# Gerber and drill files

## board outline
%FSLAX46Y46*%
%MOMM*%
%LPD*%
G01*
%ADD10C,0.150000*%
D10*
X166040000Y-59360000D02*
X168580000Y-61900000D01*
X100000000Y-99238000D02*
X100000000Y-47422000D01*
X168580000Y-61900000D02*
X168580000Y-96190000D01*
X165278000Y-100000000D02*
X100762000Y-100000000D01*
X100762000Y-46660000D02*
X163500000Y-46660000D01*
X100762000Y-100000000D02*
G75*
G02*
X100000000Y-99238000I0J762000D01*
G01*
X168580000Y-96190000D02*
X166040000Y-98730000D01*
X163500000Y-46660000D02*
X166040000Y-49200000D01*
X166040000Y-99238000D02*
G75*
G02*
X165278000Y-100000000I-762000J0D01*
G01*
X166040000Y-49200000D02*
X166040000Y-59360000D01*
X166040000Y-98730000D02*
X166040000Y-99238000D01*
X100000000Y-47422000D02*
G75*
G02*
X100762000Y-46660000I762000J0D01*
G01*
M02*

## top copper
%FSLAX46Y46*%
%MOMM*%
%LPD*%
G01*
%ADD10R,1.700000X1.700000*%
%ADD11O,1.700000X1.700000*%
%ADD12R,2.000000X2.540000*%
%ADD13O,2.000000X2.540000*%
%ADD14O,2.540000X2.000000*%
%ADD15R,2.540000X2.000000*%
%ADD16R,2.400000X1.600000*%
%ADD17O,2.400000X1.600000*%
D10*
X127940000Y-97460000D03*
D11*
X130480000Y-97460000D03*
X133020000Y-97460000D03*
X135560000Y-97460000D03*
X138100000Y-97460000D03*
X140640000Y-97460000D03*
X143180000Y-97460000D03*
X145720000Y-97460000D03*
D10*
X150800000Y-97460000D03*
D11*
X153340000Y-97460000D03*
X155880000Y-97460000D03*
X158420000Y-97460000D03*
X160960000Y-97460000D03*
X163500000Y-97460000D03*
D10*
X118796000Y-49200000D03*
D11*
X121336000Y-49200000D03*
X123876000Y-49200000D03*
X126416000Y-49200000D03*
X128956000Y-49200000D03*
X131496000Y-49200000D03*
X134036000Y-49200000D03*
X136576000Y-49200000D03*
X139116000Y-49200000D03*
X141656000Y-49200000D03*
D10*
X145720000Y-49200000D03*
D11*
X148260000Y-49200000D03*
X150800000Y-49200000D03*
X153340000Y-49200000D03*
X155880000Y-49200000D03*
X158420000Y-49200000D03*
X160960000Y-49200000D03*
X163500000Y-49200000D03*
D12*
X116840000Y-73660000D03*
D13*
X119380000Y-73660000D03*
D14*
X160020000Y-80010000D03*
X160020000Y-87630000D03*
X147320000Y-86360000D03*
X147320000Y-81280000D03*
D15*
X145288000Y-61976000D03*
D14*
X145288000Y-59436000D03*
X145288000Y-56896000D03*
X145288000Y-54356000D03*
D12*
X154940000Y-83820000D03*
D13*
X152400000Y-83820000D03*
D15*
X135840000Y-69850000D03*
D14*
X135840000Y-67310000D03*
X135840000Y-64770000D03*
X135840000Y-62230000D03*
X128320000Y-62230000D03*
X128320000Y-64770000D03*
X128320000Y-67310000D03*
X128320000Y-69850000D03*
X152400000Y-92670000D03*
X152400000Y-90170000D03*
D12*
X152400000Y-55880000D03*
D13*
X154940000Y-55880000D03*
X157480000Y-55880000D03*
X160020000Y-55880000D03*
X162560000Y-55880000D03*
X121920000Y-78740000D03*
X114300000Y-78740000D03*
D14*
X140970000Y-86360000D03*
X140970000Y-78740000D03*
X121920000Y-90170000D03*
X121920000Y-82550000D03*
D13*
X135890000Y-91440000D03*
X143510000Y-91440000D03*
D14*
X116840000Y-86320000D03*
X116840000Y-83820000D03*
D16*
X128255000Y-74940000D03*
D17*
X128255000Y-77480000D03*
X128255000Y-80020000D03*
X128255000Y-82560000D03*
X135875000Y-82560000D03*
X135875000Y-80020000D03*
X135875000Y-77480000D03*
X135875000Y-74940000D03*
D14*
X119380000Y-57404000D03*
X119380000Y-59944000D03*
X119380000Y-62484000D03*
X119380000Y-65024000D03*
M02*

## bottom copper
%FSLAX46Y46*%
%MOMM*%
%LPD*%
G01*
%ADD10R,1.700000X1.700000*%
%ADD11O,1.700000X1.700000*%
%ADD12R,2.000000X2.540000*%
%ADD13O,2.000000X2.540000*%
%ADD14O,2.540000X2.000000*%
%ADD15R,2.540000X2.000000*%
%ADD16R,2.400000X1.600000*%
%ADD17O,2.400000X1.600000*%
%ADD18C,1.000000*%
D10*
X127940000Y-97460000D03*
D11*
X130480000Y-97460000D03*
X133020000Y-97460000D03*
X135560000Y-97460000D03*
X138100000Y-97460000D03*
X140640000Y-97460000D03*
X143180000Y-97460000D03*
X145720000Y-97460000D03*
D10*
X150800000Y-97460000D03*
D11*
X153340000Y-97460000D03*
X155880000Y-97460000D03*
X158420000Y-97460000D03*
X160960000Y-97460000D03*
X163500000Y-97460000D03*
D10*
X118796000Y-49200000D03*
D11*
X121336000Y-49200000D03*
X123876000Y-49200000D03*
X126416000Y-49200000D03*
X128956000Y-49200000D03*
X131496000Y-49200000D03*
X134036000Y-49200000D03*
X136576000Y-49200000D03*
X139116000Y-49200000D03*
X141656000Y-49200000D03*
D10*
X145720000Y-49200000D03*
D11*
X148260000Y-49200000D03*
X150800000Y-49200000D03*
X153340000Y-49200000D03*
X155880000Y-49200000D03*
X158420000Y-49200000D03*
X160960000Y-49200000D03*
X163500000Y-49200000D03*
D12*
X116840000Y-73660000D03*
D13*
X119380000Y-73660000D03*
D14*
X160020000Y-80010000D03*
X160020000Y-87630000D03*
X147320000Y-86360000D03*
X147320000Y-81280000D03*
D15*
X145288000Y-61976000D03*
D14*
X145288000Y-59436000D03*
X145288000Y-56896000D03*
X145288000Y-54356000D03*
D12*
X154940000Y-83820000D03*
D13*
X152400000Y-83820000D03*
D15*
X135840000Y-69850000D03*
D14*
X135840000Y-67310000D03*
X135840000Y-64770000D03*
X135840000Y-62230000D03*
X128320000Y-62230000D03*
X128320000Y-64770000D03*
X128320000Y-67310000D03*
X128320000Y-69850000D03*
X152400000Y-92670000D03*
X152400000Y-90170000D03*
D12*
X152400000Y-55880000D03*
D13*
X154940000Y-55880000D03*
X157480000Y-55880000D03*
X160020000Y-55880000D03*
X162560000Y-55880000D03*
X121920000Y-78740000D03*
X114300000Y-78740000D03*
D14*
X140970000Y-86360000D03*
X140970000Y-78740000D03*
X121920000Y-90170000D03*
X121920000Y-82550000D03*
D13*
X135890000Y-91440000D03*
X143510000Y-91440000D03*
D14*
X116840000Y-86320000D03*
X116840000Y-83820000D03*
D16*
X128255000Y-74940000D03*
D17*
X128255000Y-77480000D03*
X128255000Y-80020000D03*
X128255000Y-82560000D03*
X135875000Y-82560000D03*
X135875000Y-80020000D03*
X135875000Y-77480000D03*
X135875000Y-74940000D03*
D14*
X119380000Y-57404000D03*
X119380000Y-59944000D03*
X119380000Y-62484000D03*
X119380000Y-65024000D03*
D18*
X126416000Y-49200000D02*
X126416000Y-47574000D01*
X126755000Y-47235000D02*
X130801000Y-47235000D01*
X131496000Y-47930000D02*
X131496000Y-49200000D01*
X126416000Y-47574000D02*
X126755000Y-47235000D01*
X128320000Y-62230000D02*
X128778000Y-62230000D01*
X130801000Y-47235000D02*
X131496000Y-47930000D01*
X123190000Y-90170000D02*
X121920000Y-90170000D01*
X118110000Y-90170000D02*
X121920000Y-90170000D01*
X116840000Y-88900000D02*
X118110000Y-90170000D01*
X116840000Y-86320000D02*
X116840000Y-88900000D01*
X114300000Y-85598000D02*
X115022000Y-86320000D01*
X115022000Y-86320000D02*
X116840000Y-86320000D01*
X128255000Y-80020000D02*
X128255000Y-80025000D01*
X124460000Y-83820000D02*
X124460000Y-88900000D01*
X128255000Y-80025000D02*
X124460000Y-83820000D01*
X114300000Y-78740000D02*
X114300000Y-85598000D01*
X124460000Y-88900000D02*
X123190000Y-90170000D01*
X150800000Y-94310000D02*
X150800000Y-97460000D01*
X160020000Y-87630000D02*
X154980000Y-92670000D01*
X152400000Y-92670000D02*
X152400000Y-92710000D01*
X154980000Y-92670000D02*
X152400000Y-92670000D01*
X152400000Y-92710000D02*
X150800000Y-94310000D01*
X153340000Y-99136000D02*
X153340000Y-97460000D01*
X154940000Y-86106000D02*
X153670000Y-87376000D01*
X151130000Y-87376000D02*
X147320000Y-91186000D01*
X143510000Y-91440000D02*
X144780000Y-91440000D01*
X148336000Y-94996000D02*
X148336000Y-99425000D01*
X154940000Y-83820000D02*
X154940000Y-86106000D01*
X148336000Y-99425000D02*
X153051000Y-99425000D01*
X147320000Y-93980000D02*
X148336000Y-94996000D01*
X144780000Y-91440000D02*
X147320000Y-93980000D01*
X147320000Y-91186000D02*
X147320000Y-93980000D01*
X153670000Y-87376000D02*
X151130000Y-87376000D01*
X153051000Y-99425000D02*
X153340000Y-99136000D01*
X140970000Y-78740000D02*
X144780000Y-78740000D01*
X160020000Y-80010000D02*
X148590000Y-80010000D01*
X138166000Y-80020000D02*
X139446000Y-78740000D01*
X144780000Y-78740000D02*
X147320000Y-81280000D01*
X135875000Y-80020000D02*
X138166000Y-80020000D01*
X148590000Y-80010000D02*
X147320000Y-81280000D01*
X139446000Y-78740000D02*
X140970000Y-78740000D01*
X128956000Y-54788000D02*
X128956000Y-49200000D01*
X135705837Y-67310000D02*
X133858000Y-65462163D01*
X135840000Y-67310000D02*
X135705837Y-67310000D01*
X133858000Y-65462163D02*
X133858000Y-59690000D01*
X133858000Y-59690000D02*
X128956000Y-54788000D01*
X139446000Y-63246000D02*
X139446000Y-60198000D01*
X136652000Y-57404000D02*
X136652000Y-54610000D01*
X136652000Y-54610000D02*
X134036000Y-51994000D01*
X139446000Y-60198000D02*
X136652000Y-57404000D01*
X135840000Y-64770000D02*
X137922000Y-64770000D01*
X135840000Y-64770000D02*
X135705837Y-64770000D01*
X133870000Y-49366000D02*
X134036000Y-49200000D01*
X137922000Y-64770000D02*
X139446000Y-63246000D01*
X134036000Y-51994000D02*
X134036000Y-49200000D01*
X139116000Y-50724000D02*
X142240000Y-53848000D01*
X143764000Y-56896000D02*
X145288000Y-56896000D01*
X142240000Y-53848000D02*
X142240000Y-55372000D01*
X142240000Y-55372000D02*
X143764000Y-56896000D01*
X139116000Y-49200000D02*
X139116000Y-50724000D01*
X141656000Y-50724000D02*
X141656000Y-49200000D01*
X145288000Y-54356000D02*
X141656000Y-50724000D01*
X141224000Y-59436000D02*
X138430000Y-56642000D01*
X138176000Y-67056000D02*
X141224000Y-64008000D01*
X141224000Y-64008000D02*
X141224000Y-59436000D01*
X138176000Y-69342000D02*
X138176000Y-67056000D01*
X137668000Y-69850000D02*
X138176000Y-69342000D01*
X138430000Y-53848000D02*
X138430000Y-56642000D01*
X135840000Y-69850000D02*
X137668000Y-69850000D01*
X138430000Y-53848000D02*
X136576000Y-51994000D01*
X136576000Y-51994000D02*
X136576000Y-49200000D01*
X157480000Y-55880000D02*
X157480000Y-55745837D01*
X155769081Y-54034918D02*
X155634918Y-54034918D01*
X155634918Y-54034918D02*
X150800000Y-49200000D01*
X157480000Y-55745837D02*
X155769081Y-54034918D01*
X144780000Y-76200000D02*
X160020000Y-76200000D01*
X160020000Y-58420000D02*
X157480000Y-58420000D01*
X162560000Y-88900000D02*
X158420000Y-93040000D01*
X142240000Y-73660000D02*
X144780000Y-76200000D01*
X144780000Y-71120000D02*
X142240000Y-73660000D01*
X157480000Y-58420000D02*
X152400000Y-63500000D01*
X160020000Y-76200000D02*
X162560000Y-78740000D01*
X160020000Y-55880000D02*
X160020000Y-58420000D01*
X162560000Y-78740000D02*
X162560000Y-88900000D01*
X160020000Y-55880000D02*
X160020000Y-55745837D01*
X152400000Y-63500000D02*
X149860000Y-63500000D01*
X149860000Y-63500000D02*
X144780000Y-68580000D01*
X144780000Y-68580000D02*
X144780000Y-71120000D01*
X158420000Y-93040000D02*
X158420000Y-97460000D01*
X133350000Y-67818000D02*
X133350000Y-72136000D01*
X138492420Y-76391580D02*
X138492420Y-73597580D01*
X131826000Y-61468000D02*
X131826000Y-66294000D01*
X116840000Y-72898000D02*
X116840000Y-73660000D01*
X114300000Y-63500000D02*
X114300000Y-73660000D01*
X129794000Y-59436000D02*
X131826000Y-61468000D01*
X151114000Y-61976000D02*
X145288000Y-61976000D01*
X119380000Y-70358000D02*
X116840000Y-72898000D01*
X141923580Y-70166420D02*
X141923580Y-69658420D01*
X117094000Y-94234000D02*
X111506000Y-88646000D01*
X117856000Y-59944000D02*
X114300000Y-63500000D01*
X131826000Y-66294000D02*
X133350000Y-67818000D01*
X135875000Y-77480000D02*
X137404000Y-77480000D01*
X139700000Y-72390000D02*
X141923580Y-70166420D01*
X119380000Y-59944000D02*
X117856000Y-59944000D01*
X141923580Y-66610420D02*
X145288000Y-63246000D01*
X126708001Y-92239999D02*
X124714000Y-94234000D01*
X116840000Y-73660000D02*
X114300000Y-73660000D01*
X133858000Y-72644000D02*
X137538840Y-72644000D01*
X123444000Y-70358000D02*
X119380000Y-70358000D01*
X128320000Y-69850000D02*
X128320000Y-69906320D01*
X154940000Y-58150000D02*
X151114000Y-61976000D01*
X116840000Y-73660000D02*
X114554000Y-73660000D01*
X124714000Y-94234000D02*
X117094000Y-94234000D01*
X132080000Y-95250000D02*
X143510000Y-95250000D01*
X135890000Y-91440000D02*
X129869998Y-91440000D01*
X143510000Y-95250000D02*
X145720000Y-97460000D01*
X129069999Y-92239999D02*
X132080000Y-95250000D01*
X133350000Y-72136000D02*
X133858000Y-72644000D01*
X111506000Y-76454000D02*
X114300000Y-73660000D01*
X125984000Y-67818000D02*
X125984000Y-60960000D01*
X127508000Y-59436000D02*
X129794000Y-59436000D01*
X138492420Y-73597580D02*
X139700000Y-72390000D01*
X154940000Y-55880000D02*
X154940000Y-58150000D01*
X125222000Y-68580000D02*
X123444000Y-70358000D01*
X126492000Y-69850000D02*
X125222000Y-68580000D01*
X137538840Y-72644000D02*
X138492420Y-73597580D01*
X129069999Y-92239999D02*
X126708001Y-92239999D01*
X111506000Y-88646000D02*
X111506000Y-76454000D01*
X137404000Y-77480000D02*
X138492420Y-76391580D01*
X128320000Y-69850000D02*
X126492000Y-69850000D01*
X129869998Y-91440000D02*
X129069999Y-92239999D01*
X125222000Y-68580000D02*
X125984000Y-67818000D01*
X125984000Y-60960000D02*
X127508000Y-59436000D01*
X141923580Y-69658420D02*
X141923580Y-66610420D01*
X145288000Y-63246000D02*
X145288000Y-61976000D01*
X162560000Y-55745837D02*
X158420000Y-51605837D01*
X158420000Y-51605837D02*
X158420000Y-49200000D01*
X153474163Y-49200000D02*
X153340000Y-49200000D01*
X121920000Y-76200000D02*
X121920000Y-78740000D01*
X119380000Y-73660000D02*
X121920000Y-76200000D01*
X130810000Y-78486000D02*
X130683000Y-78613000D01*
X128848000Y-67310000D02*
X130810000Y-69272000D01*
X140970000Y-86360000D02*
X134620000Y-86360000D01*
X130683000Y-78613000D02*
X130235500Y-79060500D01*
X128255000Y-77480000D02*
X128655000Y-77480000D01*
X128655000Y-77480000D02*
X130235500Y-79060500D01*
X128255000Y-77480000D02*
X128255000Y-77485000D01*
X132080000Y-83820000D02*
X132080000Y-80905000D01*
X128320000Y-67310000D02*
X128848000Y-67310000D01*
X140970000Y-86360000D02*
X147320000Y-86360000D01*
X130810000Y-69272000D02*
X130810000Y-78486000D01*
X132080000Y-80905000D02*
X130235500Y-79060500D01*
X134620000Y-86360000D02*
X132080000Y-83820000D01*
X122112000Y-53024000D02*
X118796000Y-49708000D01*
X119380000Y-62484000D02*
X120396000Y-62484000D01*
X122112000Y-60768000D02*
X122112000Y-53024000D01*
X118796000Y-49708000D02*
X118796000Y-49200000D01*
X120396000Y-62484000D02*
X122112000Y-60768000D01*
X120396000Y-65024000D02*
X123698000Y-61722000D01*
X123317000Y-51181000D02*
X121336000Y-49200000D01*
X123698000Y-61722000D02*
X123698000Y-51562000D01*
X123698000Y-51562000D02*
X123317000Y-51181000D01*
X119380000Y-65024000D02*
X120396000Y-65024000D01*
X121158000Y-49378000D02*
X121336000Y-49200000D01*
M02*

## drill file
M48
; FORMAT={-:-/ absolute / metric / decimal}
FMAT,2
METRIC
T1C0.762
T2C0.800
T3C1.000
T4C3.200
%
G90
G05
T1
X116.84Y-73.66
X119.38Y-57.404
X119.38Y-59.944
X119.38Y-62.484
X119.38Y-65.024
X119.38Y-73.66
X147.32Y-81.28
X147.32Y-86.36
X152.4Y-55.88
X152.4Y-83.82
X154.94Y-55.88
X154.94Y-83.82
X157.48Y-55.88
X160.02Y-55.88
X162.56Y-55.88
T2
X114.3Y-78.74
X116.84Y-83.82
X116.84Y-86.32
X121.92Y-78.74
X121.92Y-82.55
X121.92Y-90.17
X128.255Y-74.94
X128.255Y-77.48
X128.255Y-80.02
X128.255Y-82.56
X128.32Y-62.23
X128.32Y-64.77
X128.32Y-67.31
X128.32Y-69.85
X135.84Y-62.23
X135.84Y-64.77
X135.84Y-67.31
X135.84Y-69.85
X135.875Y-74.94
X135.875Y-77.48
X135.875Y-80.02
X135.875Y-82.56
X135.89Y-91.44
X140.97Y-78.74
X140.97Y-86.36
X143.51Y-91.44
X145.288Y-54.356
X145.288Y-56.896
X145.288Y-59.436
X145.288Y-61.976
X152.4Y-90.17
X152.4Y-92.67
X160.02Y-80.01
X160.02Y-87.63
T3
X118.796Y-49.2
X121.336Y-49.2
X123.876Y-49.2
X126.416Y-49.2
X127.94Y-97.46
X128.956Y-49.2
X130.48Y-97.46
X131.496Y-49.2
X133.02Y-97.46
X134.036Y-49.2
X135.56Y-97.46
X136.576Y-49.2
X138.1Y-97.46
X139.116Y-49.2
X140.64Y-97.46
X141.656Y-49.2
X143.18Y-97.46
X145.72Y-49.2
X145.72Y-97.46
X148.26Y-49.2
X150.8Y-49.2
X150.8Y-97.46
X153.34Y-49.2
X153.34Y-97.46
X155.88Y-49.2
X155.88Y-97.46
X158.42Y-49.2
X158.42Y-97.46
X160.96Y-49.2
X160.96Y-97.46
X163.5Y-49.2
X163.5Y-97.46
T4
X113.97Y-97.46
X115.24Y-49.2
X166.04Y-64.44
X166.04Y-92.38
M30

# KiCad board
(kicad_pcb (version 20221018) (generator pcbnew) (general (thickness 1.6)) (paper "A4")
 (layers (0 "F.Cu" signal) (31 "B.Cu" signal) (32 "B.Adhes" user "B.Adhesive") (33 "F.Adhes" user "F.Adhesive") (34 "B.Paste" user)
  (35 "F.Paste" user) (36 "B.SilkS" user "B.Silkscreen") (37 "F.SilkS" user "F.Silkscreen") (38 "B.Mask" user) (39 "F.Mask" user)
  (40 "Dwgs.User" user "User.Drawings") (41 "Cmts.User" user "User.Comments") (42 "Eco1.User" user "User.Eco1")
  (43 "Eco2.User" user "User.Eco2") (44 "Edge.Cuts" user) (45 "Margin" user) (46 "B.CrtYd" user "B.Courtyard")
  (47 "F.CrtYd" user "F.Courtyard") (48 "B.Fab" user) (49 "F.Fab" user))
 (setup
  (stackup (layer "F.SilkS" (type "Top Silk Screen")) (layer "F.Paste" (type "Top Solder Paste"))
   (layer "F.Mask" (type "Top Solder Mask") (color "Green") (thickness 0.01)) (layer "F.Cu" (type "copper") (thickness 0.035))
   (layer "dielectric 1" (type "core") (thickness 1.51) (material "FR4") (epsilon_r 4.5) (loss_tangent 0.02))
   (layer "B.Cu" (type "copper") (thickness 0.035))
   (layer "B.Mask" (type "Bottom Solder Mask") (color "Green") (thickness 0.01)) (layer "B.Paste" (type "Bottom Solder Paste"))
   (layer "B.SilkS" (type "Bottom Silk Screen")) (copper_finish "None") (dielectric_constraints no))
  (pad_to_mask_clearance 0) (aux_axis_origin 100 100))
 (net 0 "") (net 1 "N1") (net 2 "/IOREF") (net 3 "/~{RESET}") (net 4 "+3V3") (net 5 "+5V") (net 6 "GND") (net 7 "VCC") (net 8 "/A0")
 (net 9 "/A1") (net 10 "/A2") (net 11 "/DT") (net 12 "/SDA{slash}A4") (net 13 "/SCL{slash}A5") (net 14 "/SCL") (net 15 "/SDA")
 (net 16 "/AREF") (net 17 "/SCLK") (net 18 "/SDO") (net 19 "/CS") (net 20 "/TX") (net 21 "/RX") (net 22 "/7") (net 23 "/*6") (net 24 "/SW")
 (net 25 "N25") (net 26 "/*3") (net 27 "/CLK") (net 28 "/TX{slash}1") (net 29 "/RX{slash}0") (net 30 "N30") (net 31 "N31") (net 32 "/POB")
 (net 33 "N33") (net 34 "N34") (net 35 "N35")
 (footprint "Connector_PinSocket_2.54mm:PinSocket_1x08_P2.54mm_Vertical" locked (layer "F.Cu") (at 127.94 97.46 90)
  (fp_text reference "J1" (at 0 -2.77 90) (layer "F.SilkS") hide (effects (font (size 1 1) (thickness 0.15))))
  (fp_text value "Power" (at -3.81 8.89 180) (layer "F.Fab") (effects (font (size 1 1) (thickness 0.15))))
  (pad "1" thru_hole rect locked (at 0 0 90) (size 1.7 1.7) (drill 1) (layers "*.Cu" "*.Mask") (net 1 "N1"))
  (pad "2" thru_hole oval locked (at 0 2.54 90) (size 1.7 1.7) (drill 1) (layers "*.Cu" "*.Mask") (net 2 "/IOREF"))
  (pad "3" thru_hole oval locked (at 0 5.08 90) (size 1.7 1.7) (drill 1) (layers "*.Cu" "*.Mask") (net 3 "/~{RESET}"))
  (pad "4" thru_hole oval locked (at 0 7.62 90) (size 1.7 1.7) (drill 1) (layers "*.Cu" "*.Mask") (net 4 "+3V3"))
  (pad "5" thru_hole oval locked (at 0 10.16 90) (size 1.7 1.7) (drill 1) (layers "*.Cu" "*.Mask") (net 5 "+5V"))
  (pad "6" thru_hole oval locked (at 0 12.7 90) (size 1.7 1.7) (drill 1) (layers "*.Cu" "*.Mask") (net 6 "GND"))
  (pad "7" thru_hole oval locked (at 0 15.24 90) (size 1.7 1.7) (drill 1) (layers "*.Cu" "*.Mask") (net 6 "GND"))
  (pad "8" thru_hole oval locked (at 0 17.78 90) (size 1.7 1.7) (drill 1) (layers "*.Cu" "*.Mask") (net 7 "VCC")))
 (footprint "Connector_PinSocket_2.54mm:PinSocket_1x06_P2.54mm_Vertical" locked (layer "F.Cu") (at 150.8 97.46 90)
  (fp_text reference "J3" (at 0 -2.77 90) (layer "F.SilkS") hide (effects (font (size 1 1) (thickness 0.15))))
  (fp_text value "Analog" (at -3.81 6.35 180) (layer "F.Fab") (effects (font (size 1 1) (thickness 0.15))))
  (pad "1" thru_hole rect locked (at 0 0 90) (size 1.7 1.7) (drill 1) (layers "*.Cu" "*.Mask") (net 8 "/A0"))
  (pad "2" thru_hole oval locked (at 0 2.54 90) (size 1.7 1.7) (drill 1) (layers "*.Cu" "*.Mask") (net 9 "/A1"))
  (pad "3" thru_hole oval locked (at 0 5.08 90) (size 1.7 1.7) (drill 1) (layers "*.Cu" "*.Mask") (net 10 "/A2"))
  (pad "4" thru_hole oval locked (at 0 7.62 90) (size 1.7 1.7) (drill 1) (layers "*.Cu" "*.Mask") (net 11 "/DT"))
  (pad "5" thru_hole oval locked (at 0 10.16 90) (size 1.7 1.7) (drill 1) (layers "*.Cu" "*.Mask") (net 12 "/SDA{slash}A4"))
  (pad "6" thru_hole oval locked (at 0 12.7 90) (size 1.7 1.7) (drill 1) (layers "*.Cu" "*.Mask") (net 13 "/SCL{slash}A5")))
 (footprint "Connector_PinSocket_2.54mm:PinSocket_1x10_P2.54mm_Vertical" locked (layer "F.Cu") (at 118.796 49.2 90)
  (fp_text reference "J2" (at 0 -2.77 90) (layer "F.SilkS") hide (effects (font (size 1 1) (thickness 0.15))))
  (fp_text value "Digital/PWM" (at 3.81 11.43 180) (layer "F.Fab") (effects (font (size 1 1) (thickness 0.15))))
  (pad "1" thru_hole rect locked (at 0 0 90) (size 1.7 1.7) (drill 1) (layers "*.Cu" "*.Mask") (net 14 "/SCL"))
  (pad "2" thru_hole oval locked (at 0 2.54 90) (size 1.7 1.7) (drill 1) (layers "*.Cu" "*.Mask") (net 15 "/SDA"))
  (pad "3" thru_hole oval locked (at 0 5.08 90) (size 1.7 1.7) (drill 1) (layers "*.Cu" "*.Mask") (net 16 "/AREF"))
  (pad "4" thru_hole oval locked (at 0 7.62 90) (size 1.7 1.7) (drill 1) (layers "*.Cu" "*.Mask") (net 6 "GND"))
  (pad "5" thru_hole oval locked (at 0 10.16 90) (size 1.7 1.7) (drill 1) (layers "*.Cu" "*.Mask") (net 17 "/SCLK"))
  (pad "6" thru_hole oval locked (at 0 12.7 90) (size 1.7 1.7) (drill 1) (layers "*.Cu" "*.Mask") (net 6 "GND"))
  (pad "7" thru_hole oval locked (at 0 15.24 90) (size 1.7 1.7) (drill 1) (layers "*.Cu" "*.Mask") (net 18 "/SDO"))
  (pad "8" thru_hole oval locked (at 0 17.78 90) (size 1.7 1.7) (drill 1) (layers "*.Cu" "*.Mask") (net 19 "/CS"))
  (pad "9" thru_hole oval locked (at 0 20.32 90) (size 1.7 1.7) (drill 1) (layers "*.Cu" "*.Mask") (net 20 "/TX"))
  (pad "10" thru_hole oval locked (at 0 22.86 90) (size 1.7 1.7) (drill 1) (layers "*.Cu" "*.Mask") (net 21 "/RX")))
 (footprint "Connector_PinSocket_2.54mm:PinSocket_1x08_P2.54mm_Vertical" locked (layer "F.Cu") (at 145.72 49.2 90)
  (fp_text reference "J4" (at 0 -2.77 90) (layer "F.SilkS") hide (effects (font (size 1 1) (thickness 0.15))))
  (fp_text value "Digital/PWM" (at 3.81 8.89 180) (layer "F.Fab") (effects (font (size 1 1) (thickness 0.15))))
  (pad "1" thru_hole rect locked (at 0 0 90) (size 1.7 1.7) (drill 1) (layers "*.Cu" "*.Mask") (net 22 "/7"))
  (pad "2" thru_hole oval locked (at 0 2.54 90) (size 1.7 1.7) (drill 1) (layers "*.Cu" "*.Mask") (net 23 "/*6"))
  (pad "3" thru_hole oval locked (at 0 5.08 90) (size 1.7 1.7) (drill 1) (layers "*.Cu" "*.Mask") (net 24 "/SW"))
  (pad "4" thru_hole oval locked (at 0 7.62 90) (size 1.7 1.7) (drill 1) (layers "*.Cu" "*.Mask") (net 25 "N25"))
  (pad "5" thru_hole oval locked (at 0 10.16 90) (size 1.7 1.7) (drill 1) (layers "*.Cu" "*.Mask") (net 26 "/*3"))
  (pad "6" thru_hole oval locked (at 0 12.7 90) (size 1.7 1.7) (drill 1) (layers "*.Cu" "*.Mask") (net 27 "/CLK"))
  (pad "7" thru_hole oval locked (at 0 15.24 90) (size 1.7 1.7) (drill 1) (layers "*.Cu" "*.Mask") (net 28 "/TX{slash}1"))
  (pad "8" thru_hole oval locked (at 0 17.78 90) (size 1.7 1.7) (drill 1) (layers "*.Cu" "*.Mask") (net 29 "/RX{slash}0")))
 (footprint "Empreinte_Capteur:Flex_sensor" (layer "F.Cu") (at 119.38 71.12)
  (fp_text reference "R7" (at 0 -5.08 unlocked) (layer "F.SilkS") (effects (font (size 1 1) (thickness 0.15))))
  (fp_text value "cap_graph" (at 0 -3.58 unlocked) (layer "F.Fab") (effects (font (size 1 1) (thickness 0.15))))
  (pad "1" thru_hole rect (at -2.54 2.54) (size 2 2.54) (drill 0.762) (layers "*.Cu" "*.Mask") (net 7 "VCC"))
  (pad "2" thru_hole oval (at 0 2.54) (size 2 2.54) (drill 0.762) (layers "*.Cu" "*.Mask") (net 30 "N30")))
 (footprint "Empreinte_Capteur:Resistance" (layer "F.Cu") (at 160.02 80.01 -90)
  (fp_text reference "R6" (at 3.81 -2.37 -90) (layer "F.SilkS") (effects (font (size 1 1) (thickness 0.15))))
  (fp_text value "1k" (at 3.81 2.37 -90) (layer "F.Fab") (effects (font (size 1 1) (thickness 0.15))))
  (pad "1" thru_hole oval (at 0 0 270) (size 2 2.54) (drill 0.8) (layers "*.Cu" "*.Mask") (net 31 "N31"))
  (pad "2" thru_hole oval (at 7.62 0 270) (size 2 2.54) (drill 0.8) (layers "*.Cu" "*.Mask") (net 8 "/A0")))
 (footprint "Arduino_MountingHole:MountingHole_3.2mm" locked (layer "F.Cu") (at 115.24 49.2)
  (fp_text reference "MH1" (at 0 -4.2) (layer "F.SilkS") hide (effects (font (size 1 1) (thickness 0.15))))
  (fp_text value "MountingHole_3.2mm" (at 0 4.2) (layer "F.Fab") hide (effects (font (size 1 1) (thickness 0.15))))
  (pad "" np_thru_hole circle locked (at 0 0) (size 3.2 3.2) (drill 3.2) (layers "*.Cu" "*.Mask")))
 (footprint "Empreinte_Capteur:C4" (layer "F.Cu") (at 144.78 83.82 90)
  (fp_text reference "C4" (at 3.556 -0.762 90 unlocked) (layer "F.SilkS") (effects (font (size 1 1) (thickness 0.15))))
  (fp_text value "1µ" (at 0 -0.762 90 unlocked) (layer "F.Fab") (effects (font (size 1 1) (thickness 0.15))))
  (pad "1" thru_hole oval (at -2.54 2.54 90) (size 2 2.54) (drill 0.762) (layers "*.Cu" "*.Mask") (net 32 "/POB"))
  (pad "2" thru_hole oval (at 2.54 2.54 90) (size 2 2.54) (drill 0.762) (layers "*.Cu" "*.Mask") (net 31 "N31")))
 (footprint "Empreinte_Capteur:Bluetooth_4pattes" (layer "F.Cu") (at 145.288 58.166 90)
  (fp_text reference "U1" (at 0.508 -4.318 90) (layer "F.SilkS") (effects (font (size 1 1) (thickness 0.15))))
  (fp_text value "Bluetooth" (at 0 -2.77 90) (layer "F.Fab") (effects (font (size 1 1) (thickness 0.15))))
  (pad "1" thru_hole rect (at -3.81 0 90) (size 2 2.54) (drill 0.8) (layers "*.Cu" "*.Mask") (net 7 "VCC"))
  (pad "2" thru_hole oval (at -1.27 0 90) (size 2 2.54) (drill 0.8) (layers "*.Cu" "*.Mask") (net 6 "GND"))
  (pad "3" thru_hole oval (at 1.27 0 90) (size 2 2.54) (drill 0.8) (layers "*.Cu" "*.Mask") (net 20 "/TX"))
  (pad "4" thru_hole oval (at 3.81 0 90) (size 2 2.54) (drill 0.8) (layers "*.Cu" "*.Mask") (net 21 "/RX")))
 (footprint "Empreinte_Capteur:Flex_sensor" (layer "F.Cu") (at 152.4 86.36 180)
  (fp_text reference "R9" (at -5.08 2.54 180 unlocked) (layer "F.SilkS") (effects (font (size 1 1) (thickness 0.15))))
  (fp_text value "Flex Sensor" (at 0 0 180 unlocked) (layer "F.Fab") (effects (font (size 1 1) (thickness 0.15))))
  (pad "1" thru_hole rect (at -2.54 2.54 180) (size 2 2.54) (drill 0.762) (layers "*.Cu" "*.Mask") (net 9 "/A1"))
  (pad "2" thru_hole oval (at 0 2.54 180) (size 2 2.54) (drill 0.762) (layers "*.Cu" "*.Mask") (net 6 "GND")))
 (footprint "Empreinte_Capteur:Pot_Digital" (layer "F.Cu") (at 132.08 66.04 90)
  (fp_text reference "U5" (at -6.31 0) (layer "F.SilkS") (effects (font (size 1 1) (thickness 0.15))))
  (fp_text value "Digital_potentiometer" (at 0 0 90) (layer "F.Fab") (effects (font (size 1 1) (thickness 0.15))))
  (pad "1" thru_hole rect (at -3.81 3.76 90) (size 2 2.54) (drill 0.8) (layers "*.Cu" "*.Mask") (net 19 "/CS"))
  (pad "2" thru_hole oval (at -1.27 3.76 90) (size 2 2.54) (drill 0.8) (layers "*.Cu" "*.Mask") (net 17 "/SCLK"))
  (pad "3" thru_hole oval (at 1.27 3.76 90) (size 2 2.54) (drill 0.8) (layers "*.Cu" "*.Mask") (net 18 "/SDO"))
  (pad "4" thru_hole oval (at 3.81 3.76 90) (size 2 2.54) (drill 0.8) (layers "*.Cu" "*.Mask") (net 6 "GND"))
  (pad "5" thru_hole oval (at 3.81 -3.76 90) (size 2 2.54) (drill 0.8) (layers "*.Cu" "*.Mask") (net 6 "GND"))
  (pad "6" thru_hole oval (at 1.27 -3.76 90) (size 2 2.54) (drill 0.8) (layers "*.Cu" "*.Mask") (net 6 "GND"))
  (pad "7" thru_hole oval (at -1.27 -3.76 90) (size 2 2.54) (drill 0.8) (layers "*.Cu" "*.Mask") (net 32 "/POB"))
  (pad "8" thru_hole oval (at -3.81 -3.76 90) (size 2 2.54) (drill 0.8) (layers "*.Cu" "*.Mask") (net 7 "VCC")))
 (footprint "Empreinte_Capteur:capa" (layer "F.Cu") (at 152.4 92.67 90)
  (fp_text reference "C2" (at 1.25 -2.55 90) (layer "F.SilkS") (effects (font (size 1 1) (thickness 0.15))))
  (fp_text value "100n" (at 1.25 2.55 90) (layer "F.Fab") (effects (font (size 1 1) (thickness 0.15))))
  (pad "1" thru_hole oval (at 0 0 90) (size 2 2.54) (drill 0.8) (layers "*.Cu" "*.Mask") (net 8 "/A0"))
  (pad "2" thru_hole oval (at 2.5 0 90) (size 2 2.54) (drill 0.8) (layers "*.Cu" "*.Mask") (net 6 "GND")))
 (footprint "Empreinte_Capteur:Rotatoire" (layer "F.Cu") (at 154.94 55.88)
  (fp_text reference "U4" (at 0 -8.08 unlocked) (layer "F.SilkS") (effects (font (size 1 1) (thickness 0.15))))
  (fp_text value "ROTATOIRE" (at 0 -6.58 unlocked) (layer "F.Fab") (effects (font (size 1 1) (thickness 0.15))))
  (pad "1" thru_hole rect (at -2.54 0) (size 2 2.54) (drill 0.762) (layers "*.Cu" "*.Mask") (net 6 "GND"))
  (pad "2" thru_hole oval (at 0 0) (size 2 2.54) (drill 0.762) (layers "*.Cu" "*.Mask") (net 7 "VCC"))
  (pad "3" thru_hole oval (at 2.54 0) (size 2 2.54) (drill 0.762) (layers "*.Cu" "*.Mask") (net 24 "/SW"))
  (pad "4" thru_hole oval (at 5.08 0) (size 2 2.54) (drill 0.762) (layers "*.Cu" "*.Mask") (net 11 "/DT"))
  (pad "5" thru_hole oval (at 7.62 0) (size 2 2.54) (drill 0.762) (layers "*.Cu" "*.Mask") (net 27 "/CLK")))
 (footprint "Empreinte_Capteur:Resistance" (layer "F.Cu") (at 121.92 78.74 180)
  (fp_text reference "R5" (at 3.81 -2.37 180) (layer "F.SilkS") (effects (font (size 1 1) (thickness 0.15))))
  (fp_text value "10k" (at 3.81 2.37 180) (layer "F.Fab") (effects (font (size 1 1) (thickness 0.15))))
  (pad "1" thru_hole oval (at 0 0 180) (size 2 2.54) (drill 0.8) (layers "*.Cu" "*.Mask") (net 30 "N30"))
  (pad "2" thru_hole oval (at 7.62 0 180) (size 2 2.54) (drill 0.8) (layers "*.Cu" "*.Mask") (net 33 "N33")))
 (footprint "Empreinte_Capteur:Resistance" (layer "F.Cu") (at 140.97 86.36 90)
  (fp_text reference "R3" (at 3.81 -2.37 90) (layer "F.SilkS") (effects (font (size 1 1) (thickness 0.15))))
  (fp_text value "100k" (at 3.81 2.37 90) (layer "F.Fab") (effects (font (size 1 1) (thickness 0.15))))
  (pad "1" thru_hole oval (at 0 0 90) (size 2 2.54) (drill 0.8) (layers "*.Cu" "*.Mask") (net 32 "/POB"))
  (pad "2" thru_hole oval (at 7.62 0 90) (size 2 2.54) (drill 0.8) (layers "*.Cu" "*.Mask") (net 31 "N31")))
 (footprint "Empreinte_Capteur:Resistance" (layer "F.Cu") (at 121.92 90.17 90)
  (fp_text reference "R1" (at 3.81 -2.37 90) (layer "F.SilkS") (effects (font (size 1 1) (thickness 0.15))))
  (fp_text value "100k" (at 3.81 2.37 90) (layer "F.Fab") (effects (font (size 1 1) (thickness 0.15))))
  (pad "1" thru_hole oval (at 0 0 90) (size 2 2.54) (drill 0.8) (layers "*.Cu" "*.Mask") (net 33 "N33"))
  (pad "2" thru_hole oval (at 7.62 0 90) (size 2 2.54) (drill 0.8) (layers "*.Cu" "*.Mask") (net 6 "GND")))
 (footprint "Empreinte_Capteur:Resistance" (layer "F.Cu") (at 135.89 91.44)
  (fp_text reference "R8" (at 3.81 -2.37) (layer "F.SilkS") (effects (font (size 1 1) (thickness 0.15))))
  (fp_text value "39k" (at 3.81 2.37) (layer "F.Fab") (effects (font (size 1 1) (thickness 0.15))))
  (pad "1" thru_hole oval (at 0 0) (size 2 2.54) (drill 0.8) (layers "*.Cu" "*.Mask") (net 7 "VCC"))
  (pad "2" thru_hole oval (at 7.62 0) (size 2 2.54) (drill 0.8) (layers "*.Cu" "*.Mask") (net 9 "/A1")))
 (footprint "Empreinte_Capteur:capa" (layer "F.Cu") (at 116.84 86.32 90)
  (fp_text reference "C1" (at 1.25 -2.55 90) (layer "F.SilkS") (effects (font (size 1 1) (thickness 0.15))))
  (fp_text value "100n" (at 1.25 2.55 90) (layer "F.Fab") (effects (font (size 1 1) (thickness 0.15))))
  (pad "1" thru_hole oval (at 0 0 90) (size 2 2.54) (drill 0.8) (layers "*.Cu" "*.Mask") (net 33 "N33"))
  (pad "2" thru_hole oval (at 2.5 0 90) (size 2 2.54) (drill 0.8) (layers "*.Cu" "*.Mask") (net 6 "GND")))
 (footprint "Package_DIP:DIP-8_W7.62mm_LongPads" (layer "F.Cu") (at 128.255 74.94)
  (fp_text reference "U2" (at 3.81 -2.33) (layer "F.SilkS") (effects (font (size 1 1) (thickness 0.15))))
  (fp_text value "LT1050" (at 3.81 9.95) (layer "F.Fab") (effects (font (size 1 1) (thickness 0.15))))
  (pad "1" thru_hole rect (at 0 0) (size 2.4 1.6) (drill 0.8) (layers "*.Cu" "*.Mask") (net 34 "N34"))
  (pad "2" thru_hole oval (at 0 2.54) (size 2.4 1.6) (drill 0.8) (layers "*.Cu" "*.Mask") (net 32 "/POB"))
  (pad "3" thru_hole oval (at 0 5.08) (size 2.4 1.6) (drill 0.8) (layers "*.Cu" "*.Mask") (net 33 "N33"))
  (pad "4" thru_hole oval (at 0 7.62) (size 2.4 1.6) (drill 0.8) (layers "*.Cu" "*.Mask") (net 6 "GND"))
  (pad "5" thru_hole oval (at 7.62 7.62) (size 2.4 1.6) (drill 0.8) (layers "*.Cu" "*.Mask"))
  (pad "6" thru_hole oval (at 7.62 5.08) (size 2.4 1.6) (drill 0.8) (layers "*.Cu" "*.Mask") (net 31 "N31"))
  (pad "7" thru_hole oval (at 7.62 2.54) (size 2.4 1.6) (drill 0.8) (layers "*.Cu" "*.Mask") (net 7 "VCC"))
  (pad "8" thru_hole oval (at 7.62 0) (size 2.4 1.6) (drill 0.8) (layers "*.Cu" "*.Mask") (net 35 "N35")))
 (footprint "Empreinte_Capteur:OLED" (layer "F.Cu") (at 119.38 62.484 -90)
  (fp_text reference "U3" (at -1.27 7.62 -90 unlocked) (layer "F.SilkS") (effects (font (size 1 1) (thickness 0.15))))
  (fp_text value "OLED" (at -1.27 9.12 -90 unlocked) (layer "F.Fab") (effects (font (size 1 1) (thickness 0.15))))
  (pad "1" thru_hole oval (at -5.08 0 270) (size 2 2.54) (drill 0.762) (layers "*.Cu" "*.Mask") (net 6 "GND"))
  (pad "2" thru_hole oval (at -2.54 0 270) (size 2 2.54) (drill 0.762) (layers "*.Cu" "*.Mask") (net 7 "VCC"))
  (pad "3" thru_hole oval (at 0 0 270) (size 2 2.54) (drill 0.762) (layers "*.Cu" "*.Mask") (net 14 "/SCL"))
  (pad "4" thru_hole oval (at 2.54 0 270) (size 2 2.54) (drill 0.762) (layers "*.Cu" "*.Mask") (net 15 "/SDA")))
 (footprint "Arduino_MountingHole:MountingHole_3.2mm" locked (layer "F.Cu") (at 113.97 97.46)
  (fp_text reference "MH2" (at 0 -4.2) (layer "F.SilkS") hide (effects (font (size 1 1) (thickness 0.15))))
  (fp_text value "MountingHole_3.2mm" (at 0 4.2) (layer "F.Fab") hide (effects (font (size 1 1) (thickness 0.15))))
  (pad "" np_thru_hole circle locked (at 0 0) (size 3.2 3.2) (drill 3.2) (layers "*.Cu" "*.Mask")))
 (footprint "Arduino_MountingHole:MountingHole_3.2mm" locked (layer "F.Cu") (at 166.04 64.44)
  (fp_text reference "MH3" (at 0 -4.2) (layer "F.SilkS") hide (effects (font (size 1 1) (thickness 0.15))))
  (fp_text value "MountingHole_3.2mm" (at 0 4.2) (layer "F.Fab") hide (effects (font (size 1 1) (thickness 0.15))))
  (pad "" np_thru_hole circle locked (at 0 0) (size 3.2 3.2) (drill 3.2) (layers "*.Cu" "*.Mask")))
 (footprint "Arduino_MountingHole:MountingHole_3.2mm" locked (layer "F.Cu") (at 166.04 92.38)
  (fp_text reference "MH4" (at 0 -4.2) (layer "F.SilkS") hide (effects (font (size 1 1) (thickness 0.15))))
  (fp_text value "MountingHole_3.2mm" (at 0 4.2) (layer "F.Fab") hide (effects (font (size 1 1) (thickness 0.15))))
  (pad "" np_thru_hole circle locked (at 0 0) (size 3.2 3.2) (drill 3.2) (layers "*.Cu" "*.Mask")))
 (gr_line (start 166.04 59.36) (end 168.58 61.9) (stroke (width 0.15) (type solid)) (layer "Edge.Cuts"))
 (gr_line (start 100 99.238) (end 100 47.422) (stroke (width 0.15) (type solid)) (layer "Edge.Cuts"))
 (gr_line (start 168.58 61.9) (end 168.58 96.19) (stroke (width 0.15) (type solid)) (layer "Edge.Cuts"))
 (gr_line (start 165.278 100) (end 100.762 100) (stroke (width 0.15) (type solid)) (layer "Edge.Cuts"))
 (gr_line (start 100.762 46.66) (end 163.5 46.66) (stroke (width 0.15) (type solid)) (layer "Edge.Cuts"))
 (gr_arc (start 100.762 100) (mid 100.223185 99.776815) (end 100 99.238) (stroke (width 0.15) (type solid)) (layer "Edge.Cuts"))
 (gr_line (start 168.58 96.19) (end 166.04 98.73) (stroke (width 0.15) (type solid)) (layer "Edge.Cuts"))
 (gr_line (start 163.5 46.66) (end 166.04 49.2) (stroke (width 0.15) (type solid)) (layer "Edge.Cuts"))
 (gr_arc (start 166.04 99.238) (mid 165.816815 99.776815) (end 165.278 100) (stroke (width 0.15) (type solid)) (layer "Edge.Cuts"))
 (gr_line (start 166.04 49.2) (end 166.04 59.36) (stroke (width 0.15) (type solid)) (layer "Edge.Cuts"))
 (gr_line (start 166.04 98.73) (end 166.04 99.238) (stroke (width 0.15) (type solid)) (layer "Edge.Cuts"))
 (gr_arc (start 100 47.422) (mid 100.223185 46.883185) (end 100.762 46.66) (stroke (width 0.15) (type solid)) (layer "Edge.Cuts"))
 (segment (start 126.416 49.2) (end 126.416 47.574) (width 1) (layer "B.Cu") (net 6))
 (segment (start 126.755 47.235) (end 130.801 47.235) (width 1) (layer "B.Cu") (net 6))
 (segment (start 131.496 47.93) (end 131.496 49.2) (width 1) (layer "B.Cu") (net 6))
 (segment (start 126.416 47.574) (end 126.755 47.235) (width 1) (layer "B.Cu") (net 6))
 (segment (start 128.32 62.23) (end 128.778 62.23) (width 1) (layer "B.Cu") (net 6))
 (segment (start 130.801 47.235) (end 131.496 47.93) (width 1) (layer "B.Cu") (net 6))
 (segment (start 123.19 90.17) (end 121.92 90.17) (width 1) (layer "B.Cu") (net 33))
 (segment (start 118.11 90.17) (end 121.92 90.17) (width 1) (layer "B.Cu") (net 33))
 (segment (start 116.84 88.9) (end 118.11 90.17) (width 1) (layer "B.Cu") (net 33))
 (segment (start 116.84 86.32) (end 116.84 88.9) (width 1) (layer "B.Cu") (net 33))
 (segment (start 114.3 85.598) (end 115.022 86.32) (width 1) (layer "B.Cu") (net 33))
 (segment (start 115.022 86.32) (end 116.84 86.32) (width 1) (layer "B.Cu") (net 33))
 (segment (start 128.255 80.02) (end 128.255 80.025) (width 1) (layer "B.Cu") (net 33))
 (segment (start 124.46 83.82) (end 124.46 88.9) (width 1) (layer "B.Cu") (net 33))
 (segment (start 128.255 80.025) (end 124.46 83.82) (width 1) (layer "B.Cu") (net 33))
 (segment (start 114.3 78.74) (end 114.3 85.598) (width 1) (layer "B.Cu") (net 33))
 (segment (start 124.46 88.9) (end 123.19 90.17) (width 1) (layer "B.Cu") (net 33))
 (segment (start 150.8 94.31) (end 150.8 97.46) (width 1) (layer "B.Cu") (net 8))
 (segment (start 160.02 87.63) (end 154.98 92.67) (width 1) (layer "B.Cu") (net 8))
 (segment (start 152.4 92.67) (end 152.4 92.71) (width 1) (layer "B.Cu") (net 8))
 (segment (start 154.98 92.67) (end 152.4 92.67) (width 1) (layer "B.Cu") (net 8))
 (segment (start 152.4 92.71) (end 150.8 94.31) (width 1) (layer "B.Cu") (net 8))
 (segment (start 153.34 99.136) (end 153.34 97.46) (width 1) (layer "B.Cu") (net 9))
 (segment (start 154.94 86.106) (end 153.67 87.376) (width 1) (layer "B.Cu") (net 9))
 (segment (start 151.13 87.376) (end 147.32 91.186) (width 1) (layer "B.Cu") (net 9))
 (segment (start 143.51 91.44) (end 144.78 91.44) (width 1) (layer "B.Cu") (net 9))
 (segment (start 148.336 94.996) (end 148.336 99.425) (width 1) (layer "B.Cu") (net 9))
 (segment (start 154.94 83.82) (end 154.94 86.106) (width 1) (layer "B.Cu") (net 9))
 (segment (start 148.336 99.425) (end 153.051 99.425) (width 1) (layer "B.Cu") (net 9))
 (segment (start 147.32 93.98) (end 148.336 94.996) (width 1) (layer "B.Cu") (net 9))
 (segment (start 144.78 91.44) (end 147.32 93.98) (width 1) (layer "B.Cu") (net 9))
 (segment (start 147.32 91.186) (end 147.32 93.98) (width 1) (layer "B.Cu") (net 9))
 (segment (start 153.67 87.376) (end 151.13 87.376) (width 1) (layer "B.Cu") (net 9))
 (segment (start 153.051 99.425) (end 153.34 99.136) (width 1) (layer "B.Cu") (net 9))
 (segment (start 140.97 78.74) (end 144.78 78.74) (width 1) (layer "B.Cu") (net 31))
 (segment (start 160.02 80.01) (end 148.59 80.01) (width 1) (layer "B.Cu") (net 31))
 (segment (start 138.166 80.02) (end 139.446 78.74) (width 1) (layer "B.Cu") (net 31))
 (segment (start 144.78 78.74) (end 147.32 81.28) (width 1) (layer "B.Cu") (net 31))
 (segment (start 135.875 80.02) (end 138.166 80.02) (width 1) (layer "B.Cu") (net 31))
 (segment (start 148.59 80.01) (end 147.32 81.28) (width 1) (layer "B.Cu") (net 31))
 (segment (start 139.446 78.74) (end 140.97 78.74) (width 1) (layer "B.Cu") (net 31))
 (segment (start 128.956 54.788) (end 128.956 49.2) (width 1) (layer "B.Cu") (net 17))
 (segment (start 135.705837 67.31) (end 133.858 65.462163) (width 1) (layer "B.Cu") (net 17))
 (segment (start 135.84 67.31) (end 135.705837 67.31) (width 1) (layer "B.Cu") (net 17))
 (segment (start 133.858 65.462163) (end 133.858 59.69) (width 1) (layer "B.Cu") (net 17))
 (segment (start 133.858 59.69) (end 128.956 54.788) (width 1) (layer "B.Cu") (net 17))
 (segment (start 139.446 63.246) (end 139.446 60.198) (width 1) (layer "B.Cu") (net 18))
 (segment (start 136.652 57.404) (end 136.652 54.61) (width 1) (layer "B.Cu") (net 18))
 (segment (start 136.652 54.61) (end 134.036 51.994) (width 1) (layer "B.Cu") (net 18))
 (segment (start 139.446 60.198) (end 136.652 57.404) (width 1) (layer "B.Cu") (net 18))
 (segment (start 135.84 64.77) (end 137.922 64.77) (width 1) (layer "B.Cu") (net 18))
 (segment (start 135.84 64.77) (end 135.705837 64.77) (width 1) (layer "B.Cu") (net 18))
 (segment (start 133.87 49.366) (end 134.036 49.2) (width 1) (layer "B.Cu") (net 18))
 (segment (start 137.922 64.77) (end 139.446 63.246) (width 1) (layer "B.Cu") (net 18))
 (segment (start 134.036 51.994) (end 134.036 49.2) (width 1) (layer "B.Cu") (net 18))
 (segment (start 139.116 50.724) (end 142.24 53.848) (width 1) (layer "B.Cu") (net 20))
 (segment (start 143.764 56.896) (end 145.288 56.896) (width 1) (layer "B.Cu") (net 20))
 (segment (start 142.24 53.848) (end 142.24 55.372) (width 1) (layer "B.Cu") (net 20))
 (segment (start 142.24 55.372) (end 143.764 56.896) (width 1) (layer "B.Cu") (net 20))
 (segment (start 139.116 49.2) (end 139.116 50.724) (width 1) (layer "B.Cu") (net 20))
 (segment (start 141.656 50.724) (end 141.656 49.2) (width 1) (layer "B.Cu") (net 21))
 (segment (start 145.288 54.356) (end 141.656 50.724) (width 1) (layer "B.Cu") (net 21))
 (segment (start 141.224 59.436) (end 138.43 56.642) (width 1) (layer "B.Cu") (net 19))
 (segment (start 138.176 67.056) (end 141.224 64.008) (width 1) (layer "B.Cu") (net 19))
 (segment (start 141.224 64.008) (end 141.224 59.436) (width 1) (layer "B.Cu") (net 19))
 (segment (start 138.176 69.342) (end 138.176 67.056) (width 1) (layer "B.Cu") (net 19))
 (segment (start 137.668 69.85) (end 138.176 69.342) (width 1) (layer "B.Cu") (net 19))
 (segment (start 138.43 53.848) (end 138.43 56.642) (width 1) (layer "B.Cu") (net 19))
 (segment (start 135.84 69.85) (end 137.668 69.85) (width 1) (layer "B.Cu") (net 19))
 (segment (start 138.43 53.848) (end 136.576 51.994) (width 1) (layer "B.Cu") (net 19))
 (segment (start 136.576 51.994) (end 136.576 49.2) (width 1) (layer "B.Cu") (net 19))
 (segment (start 157.48 55.88) (end 157.48 55.745837) (width 1) (layer "B.Cu") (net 24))
 (segment (start 155.769081 54.034918) (end 155.634918 54.034918) (width 1) (layer "B.Cu") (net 24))
 (segment (start 155.634918 54.034918) (end 150.8 49.2) (width 1) (layer "B.Cu") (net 24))
 (segment (start 157.48 55.745837) (end 155.769081 54.034918) (width 1) (layer "B.Cu") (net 24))
 (segment (start 144.78 76.2) (end 160.02 76.2) (width 1) (layer "B.Cu") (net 11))
 (segment (start 160.02 58.42) (end 157.48 58.42) (width 1) (layer "B.Cu") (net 11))
 (segment (start 162.56 88.9) (end 158.42 93.04) (width 1) (layer "B.Cu") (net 11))
 (segment (start 142.24 73.66) (end 144.78 76.2) (width 1) (layer "B.Cu") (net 11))
 (segment (start 144.78 71.12) (end 142.24 73.66) (width 1) (layer "B.Cu") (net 11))
 (segment (start 157.48 58.42) (end 152.4 63.5) (width 1) (layer "B.Cu") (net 11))
 (segment (start 160.02 76.2) (end 162.56 78.74) (width 1) (layer "B.Cu") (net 11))
 (segment (start 160.02 55.88) (end 160.02 58.42) (width 1) (layer "B.Cu") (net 11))
 (segment (start 162.56 78.74) (end 162.56 88.9) (width 1) (layer "B.Cu") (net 11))
 (segment (start 160.02 55.88) (end 160.02 55.745837) (width 1) (layer "B.Cu") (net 11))
 (segment (start 152.4 63.5) (end 149.86 63.5) (width 1) (layer "B.Cu") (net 11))
 (segment (start 149.86 63.5) (end 144.78 68.58) (width 1) (layer "B.Cu") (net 11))
 (segment (start 144.78 68.58) (end 144.78 71.12) (width 1) (layer "B.Cu") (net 11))
 (segment (start 158.42 93.04) (end 158.42 97.46) (width 1) (layer "B.Cu") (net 11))
 (segment (start 133.35 67.818) (end 133.35 72.136) (width 1) (layer "B.Cu") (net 7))
 (segment (start 138.49242 76.39158) (end 138.49242 73.59758) (width 1) (layer "B.Cu") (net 7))
 (segment (start 131.826 61.468) (end 131.826 66.294) (width 1) (layer "B.Cu") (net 7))
 (segment (start 116.84 72.898) (end 116.84 73.66) (width 1) (layer "B.Cu") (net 7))
 (segment (start 114.3 63.5) (end 114.3 73.66) (width 1) (layer "B.Cu") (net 7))
 (segment (start 129.794 59.436) (end 131.826 61.468) (width 1) (layer "B.Cu") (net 7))
 (segment (start 151.114 61.976) (end 145.288 61.976) (width 1) (layer "B.Cu") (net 7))
 (segment (start 119.38 70.358) (end 116.84 72.898) (width 1) (layer "B.Cu") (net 7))
 (segment (start 141.92358 70.16642) (end 141.92358 69.65842) (width 1) (layer "B.Cu") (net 7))
 (segment (start 117.094 94.234) (end 111.506 88.646) (width 1) (layer "B.Cu") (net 7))
 (segment (start 117.856 59.944) (end 114.3 63.5) (width 1) (layer "B.Cu") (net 7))
 (segment (start 131.826 66.294) (end 133.35 67.818) (width 1) (layer "B.Cu") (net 7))
 (segment (start 135.875 77.48) (end 137.404 77.48) (width 1) (layer "B.Cu") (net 7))
 (segment (start 139.7 72.39) (end 141.92358 70.16642) (width 1) (layer "B.Cu") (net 7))
 (segment (start 119.38 59.944) (end 117.856 59.944) (width 1) (layer "B.Cu") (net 7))
 (segment (start 141.92358 66.61042) (end 145.288 63.246) (width 1) (layer "B.Cu") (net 7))
 (segment (start 126.708001 92.239999) (end 124.714 94.234) (width 1) (layer "B.Cu") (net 7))
 (segment (start 116.84 73.66) (end 114.3 73.66) (width 1) (layer "B.Cu") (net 7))
 (segment (start 133.858 72.644) (end 137.53884 72.644) (width 1) (layer "B.Cu") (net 7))
 (segment (start 123.444 70.358) (end 119.38 70.358) (width 1) (layer "B.Cu") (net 7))
 (segment (start 128.32 69.85) (end 128.32 69.90632) (width 1) (layer "B.Cu") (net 7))
 (segment (start 154.94 58.15) (end 151.114 61.976) (width 1) (layer "B.Cu") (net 7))
 (segment (start 116.84 73.66) (end 114.554 73.66) (width 1) (layer "B.Cu") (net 7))
 (segment (start 124.714 94.234) (end 117.094 94.234) (width 1) (layer "B.Cu") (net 7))
 (segment (start 132.08 95.25) (end 143.51 95.25) (width 1) (layer "B.Cu") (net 7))
 (segment (start 135.89 91.44) (end 129.869998 91.44) (width 1) (layer "B.Cu") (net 7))
 (segment (start 143.51 95.25) (end 145.72 97.46) (width 1) (layer "B.Cu") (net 7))
 (segment (start 129.069999 92.239999) (end 132.08 95.25) (width 1) (layer "B.Cu") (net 7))
 (segment (start 133.35 72.136) (end 133.858 72.644) (width 1) (layer "B.Cu") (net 7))
 (segment (start 111.506 76.454) (end 114.3 73.66) (width 1) (layer "B.Cu") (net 7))
 (segment (start 125.984 67.818) (end 125.984 60.96) (width 1) (layer "B.Cu") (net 7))
 (segment (start 127.508 59.436) (end 129.794 59.436) (width 1) (layer "B.Cu") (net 7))
 (segment (start 138.49242 73.59758) (end 139.7 72.39) (width 1) (layer "B.Cu") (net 7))
 (segment (start 154.94 55.88) (end 154.94 58.15) (width 1) (layer "B.Cu") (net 7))
 (segment (start 125.222 68.58) (end 123.444 70.358) (width 1) (layer "B.Cu") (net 7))
 (segment (start 126.492 69.85) (end 125.222 68.58) (width 1) (layer "B.Cu") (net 7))
 (segment (start 137.53884 72.644) (end 138.49242 73.59758) (width 1) (layer "B.Cu") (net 7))
 (segment (start 129.069999 92.239999) (end 126.708001 92.239999) (width 1) (layer "B.Cu") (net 7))
 (segment (start 111.506 88.646) (end 111.506 76.454) (width 1) (layer "B.Cu") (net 7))
 (segment (start 137.404 77.48) (end 138.49242 76.39158) (width 1) (layer "B.Cu") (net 7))
 (segment (start 128.32 69.85) (end 126.492 69.85) (width 1) (layer "B.Cu") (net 7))
 (segment (start 129.869998 91.44) (end 129.069999 92.239999) (width 1) (layer "B.Cu") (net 7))
 (segment (start 125.222 68.58) (end 125.984 67.818) (width 1) (layer "B.Cu") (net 7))
 (segment (start 125.984 60.96) (end 127.508 59.436) (width 1) (layer "B.Cu") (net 7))
 (segment (start 141.92358 69.65842) (end 141.92358 66.61042) (width 1) (layer "B.Cu") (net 7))
 (segment (start 145.288 63.246) (end 145.288 61.976) (width 1) (layer "B.Cu") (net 7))
 (segment (start 162.56 55.745837) (end 158.42 51.605837) (width 1) (layer "B.Cu") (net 27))
 (segment (start 158.42 51.605837) (end 158.42 49.2) (width 1) (layer "B.Cu") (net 27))
 (segment (start 153.474163 49.2) (end 153.34 49.2) (width 1) (layer "B.Cu") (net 25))
 (segment (start 121.92 76.2) (end 121.92 78.74) (width 1) (layer "B.Cu") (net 30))
 (segment (start 119.38 73.66) (end 121.92 76.2) (width 1) (layer "B.Cu") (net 30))
 (segment (start 130.81 78.486) (end 130.683 78.613) (width 1) (layer "B.Cu") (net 32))
 (segment (start 128.848 67.31) (end 130.81 69.272) (width 1) (layer "B.Cu") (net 32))
 (segment (start 140.97 86.36) (end 134.62 86.36) (width 1) (layer "B.Cu") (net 32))
 (segment (start 130.683 78.613) (end 130.2355 79.0605) (width 1) (layer "B.Cu") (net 32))
 (segment (start 128.255 77.48) (end 128.655 77.48) (width 1) (layer "B.Cu") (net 32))
 (segment (start 128.655 77.48) (end 130.2355 79.0605) (width 1) (layer "B.Cu") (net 32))
 (segment (start 128.255 77.48) (end 128.255 77.485) (width 1) (layer "B.Cu") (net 32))
 (segment (start 132.08 83.82) (end 132.08 80.905) (width 1) (layer "B.Cu") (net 32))
 (segment (start 128.32 67.31) (end 128.848 67.31) (width 1) (layer "B.Cu") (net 32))
 (segment (start 140.97 86.36) (end 147.32 86.36) (width 1) (layer "B.Cu") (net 32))
 (segment (start 130.81 69.272) (end 130.81 78.486) (width 1) (layer "B.Cu") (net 32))
 (segment (start 132.08 80.905) (end 130.2355 79.0605) (width 1) (layer "B.Cu") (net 32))
 (segment (start 134.62 86.36) (end 132.08 83.82) (width 1) (layer "B.Cu") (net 32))
 (segment (start 122.112 53.024) (end 118.796 49.708) (width 1) (layer "B.Cu") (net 14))
 (segment (start 119.38 62.484) (end 120.396 62.484) (width 1) (layer "B.Cu") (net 14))
 (segment (start 122.112 60.768) (end 122.112 53.024) (width 1) (layer "B.Cu") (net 14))
 (segment (start 118.796 49.708) (end 118.796 49.2) (width 1) (layer "B.Cu") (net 14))
 (segment (start 120.396 62.484) (end 122.112 60.768) (width 1) (layer "B.Cu") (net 14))
 (segment (start 120.396 65.024) (end 123.698 61.722) (width 1) (layer "B.Cu") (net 15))
 (segment (start 123.317 51.181) (end 121.336 49.2) (width 1) (layer "B.Cu") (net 15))
 (segment (start 123.698 61.722) (end 123.698 51.562) (width 1) (layer "B.Cu") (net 15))
 (segment (start 123.698 51.562) (end 123.317 51.181) (width 1) (layer "B.Cu") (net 15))
 (segment (start 119.38 65.024) (end 120.396 65.024) (width 1) (layer "B.Cu") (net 15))
 (segment (start 121.158 49.378) (end 121.336 49.2) (width 1) (layer "B.Cu") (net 15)))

